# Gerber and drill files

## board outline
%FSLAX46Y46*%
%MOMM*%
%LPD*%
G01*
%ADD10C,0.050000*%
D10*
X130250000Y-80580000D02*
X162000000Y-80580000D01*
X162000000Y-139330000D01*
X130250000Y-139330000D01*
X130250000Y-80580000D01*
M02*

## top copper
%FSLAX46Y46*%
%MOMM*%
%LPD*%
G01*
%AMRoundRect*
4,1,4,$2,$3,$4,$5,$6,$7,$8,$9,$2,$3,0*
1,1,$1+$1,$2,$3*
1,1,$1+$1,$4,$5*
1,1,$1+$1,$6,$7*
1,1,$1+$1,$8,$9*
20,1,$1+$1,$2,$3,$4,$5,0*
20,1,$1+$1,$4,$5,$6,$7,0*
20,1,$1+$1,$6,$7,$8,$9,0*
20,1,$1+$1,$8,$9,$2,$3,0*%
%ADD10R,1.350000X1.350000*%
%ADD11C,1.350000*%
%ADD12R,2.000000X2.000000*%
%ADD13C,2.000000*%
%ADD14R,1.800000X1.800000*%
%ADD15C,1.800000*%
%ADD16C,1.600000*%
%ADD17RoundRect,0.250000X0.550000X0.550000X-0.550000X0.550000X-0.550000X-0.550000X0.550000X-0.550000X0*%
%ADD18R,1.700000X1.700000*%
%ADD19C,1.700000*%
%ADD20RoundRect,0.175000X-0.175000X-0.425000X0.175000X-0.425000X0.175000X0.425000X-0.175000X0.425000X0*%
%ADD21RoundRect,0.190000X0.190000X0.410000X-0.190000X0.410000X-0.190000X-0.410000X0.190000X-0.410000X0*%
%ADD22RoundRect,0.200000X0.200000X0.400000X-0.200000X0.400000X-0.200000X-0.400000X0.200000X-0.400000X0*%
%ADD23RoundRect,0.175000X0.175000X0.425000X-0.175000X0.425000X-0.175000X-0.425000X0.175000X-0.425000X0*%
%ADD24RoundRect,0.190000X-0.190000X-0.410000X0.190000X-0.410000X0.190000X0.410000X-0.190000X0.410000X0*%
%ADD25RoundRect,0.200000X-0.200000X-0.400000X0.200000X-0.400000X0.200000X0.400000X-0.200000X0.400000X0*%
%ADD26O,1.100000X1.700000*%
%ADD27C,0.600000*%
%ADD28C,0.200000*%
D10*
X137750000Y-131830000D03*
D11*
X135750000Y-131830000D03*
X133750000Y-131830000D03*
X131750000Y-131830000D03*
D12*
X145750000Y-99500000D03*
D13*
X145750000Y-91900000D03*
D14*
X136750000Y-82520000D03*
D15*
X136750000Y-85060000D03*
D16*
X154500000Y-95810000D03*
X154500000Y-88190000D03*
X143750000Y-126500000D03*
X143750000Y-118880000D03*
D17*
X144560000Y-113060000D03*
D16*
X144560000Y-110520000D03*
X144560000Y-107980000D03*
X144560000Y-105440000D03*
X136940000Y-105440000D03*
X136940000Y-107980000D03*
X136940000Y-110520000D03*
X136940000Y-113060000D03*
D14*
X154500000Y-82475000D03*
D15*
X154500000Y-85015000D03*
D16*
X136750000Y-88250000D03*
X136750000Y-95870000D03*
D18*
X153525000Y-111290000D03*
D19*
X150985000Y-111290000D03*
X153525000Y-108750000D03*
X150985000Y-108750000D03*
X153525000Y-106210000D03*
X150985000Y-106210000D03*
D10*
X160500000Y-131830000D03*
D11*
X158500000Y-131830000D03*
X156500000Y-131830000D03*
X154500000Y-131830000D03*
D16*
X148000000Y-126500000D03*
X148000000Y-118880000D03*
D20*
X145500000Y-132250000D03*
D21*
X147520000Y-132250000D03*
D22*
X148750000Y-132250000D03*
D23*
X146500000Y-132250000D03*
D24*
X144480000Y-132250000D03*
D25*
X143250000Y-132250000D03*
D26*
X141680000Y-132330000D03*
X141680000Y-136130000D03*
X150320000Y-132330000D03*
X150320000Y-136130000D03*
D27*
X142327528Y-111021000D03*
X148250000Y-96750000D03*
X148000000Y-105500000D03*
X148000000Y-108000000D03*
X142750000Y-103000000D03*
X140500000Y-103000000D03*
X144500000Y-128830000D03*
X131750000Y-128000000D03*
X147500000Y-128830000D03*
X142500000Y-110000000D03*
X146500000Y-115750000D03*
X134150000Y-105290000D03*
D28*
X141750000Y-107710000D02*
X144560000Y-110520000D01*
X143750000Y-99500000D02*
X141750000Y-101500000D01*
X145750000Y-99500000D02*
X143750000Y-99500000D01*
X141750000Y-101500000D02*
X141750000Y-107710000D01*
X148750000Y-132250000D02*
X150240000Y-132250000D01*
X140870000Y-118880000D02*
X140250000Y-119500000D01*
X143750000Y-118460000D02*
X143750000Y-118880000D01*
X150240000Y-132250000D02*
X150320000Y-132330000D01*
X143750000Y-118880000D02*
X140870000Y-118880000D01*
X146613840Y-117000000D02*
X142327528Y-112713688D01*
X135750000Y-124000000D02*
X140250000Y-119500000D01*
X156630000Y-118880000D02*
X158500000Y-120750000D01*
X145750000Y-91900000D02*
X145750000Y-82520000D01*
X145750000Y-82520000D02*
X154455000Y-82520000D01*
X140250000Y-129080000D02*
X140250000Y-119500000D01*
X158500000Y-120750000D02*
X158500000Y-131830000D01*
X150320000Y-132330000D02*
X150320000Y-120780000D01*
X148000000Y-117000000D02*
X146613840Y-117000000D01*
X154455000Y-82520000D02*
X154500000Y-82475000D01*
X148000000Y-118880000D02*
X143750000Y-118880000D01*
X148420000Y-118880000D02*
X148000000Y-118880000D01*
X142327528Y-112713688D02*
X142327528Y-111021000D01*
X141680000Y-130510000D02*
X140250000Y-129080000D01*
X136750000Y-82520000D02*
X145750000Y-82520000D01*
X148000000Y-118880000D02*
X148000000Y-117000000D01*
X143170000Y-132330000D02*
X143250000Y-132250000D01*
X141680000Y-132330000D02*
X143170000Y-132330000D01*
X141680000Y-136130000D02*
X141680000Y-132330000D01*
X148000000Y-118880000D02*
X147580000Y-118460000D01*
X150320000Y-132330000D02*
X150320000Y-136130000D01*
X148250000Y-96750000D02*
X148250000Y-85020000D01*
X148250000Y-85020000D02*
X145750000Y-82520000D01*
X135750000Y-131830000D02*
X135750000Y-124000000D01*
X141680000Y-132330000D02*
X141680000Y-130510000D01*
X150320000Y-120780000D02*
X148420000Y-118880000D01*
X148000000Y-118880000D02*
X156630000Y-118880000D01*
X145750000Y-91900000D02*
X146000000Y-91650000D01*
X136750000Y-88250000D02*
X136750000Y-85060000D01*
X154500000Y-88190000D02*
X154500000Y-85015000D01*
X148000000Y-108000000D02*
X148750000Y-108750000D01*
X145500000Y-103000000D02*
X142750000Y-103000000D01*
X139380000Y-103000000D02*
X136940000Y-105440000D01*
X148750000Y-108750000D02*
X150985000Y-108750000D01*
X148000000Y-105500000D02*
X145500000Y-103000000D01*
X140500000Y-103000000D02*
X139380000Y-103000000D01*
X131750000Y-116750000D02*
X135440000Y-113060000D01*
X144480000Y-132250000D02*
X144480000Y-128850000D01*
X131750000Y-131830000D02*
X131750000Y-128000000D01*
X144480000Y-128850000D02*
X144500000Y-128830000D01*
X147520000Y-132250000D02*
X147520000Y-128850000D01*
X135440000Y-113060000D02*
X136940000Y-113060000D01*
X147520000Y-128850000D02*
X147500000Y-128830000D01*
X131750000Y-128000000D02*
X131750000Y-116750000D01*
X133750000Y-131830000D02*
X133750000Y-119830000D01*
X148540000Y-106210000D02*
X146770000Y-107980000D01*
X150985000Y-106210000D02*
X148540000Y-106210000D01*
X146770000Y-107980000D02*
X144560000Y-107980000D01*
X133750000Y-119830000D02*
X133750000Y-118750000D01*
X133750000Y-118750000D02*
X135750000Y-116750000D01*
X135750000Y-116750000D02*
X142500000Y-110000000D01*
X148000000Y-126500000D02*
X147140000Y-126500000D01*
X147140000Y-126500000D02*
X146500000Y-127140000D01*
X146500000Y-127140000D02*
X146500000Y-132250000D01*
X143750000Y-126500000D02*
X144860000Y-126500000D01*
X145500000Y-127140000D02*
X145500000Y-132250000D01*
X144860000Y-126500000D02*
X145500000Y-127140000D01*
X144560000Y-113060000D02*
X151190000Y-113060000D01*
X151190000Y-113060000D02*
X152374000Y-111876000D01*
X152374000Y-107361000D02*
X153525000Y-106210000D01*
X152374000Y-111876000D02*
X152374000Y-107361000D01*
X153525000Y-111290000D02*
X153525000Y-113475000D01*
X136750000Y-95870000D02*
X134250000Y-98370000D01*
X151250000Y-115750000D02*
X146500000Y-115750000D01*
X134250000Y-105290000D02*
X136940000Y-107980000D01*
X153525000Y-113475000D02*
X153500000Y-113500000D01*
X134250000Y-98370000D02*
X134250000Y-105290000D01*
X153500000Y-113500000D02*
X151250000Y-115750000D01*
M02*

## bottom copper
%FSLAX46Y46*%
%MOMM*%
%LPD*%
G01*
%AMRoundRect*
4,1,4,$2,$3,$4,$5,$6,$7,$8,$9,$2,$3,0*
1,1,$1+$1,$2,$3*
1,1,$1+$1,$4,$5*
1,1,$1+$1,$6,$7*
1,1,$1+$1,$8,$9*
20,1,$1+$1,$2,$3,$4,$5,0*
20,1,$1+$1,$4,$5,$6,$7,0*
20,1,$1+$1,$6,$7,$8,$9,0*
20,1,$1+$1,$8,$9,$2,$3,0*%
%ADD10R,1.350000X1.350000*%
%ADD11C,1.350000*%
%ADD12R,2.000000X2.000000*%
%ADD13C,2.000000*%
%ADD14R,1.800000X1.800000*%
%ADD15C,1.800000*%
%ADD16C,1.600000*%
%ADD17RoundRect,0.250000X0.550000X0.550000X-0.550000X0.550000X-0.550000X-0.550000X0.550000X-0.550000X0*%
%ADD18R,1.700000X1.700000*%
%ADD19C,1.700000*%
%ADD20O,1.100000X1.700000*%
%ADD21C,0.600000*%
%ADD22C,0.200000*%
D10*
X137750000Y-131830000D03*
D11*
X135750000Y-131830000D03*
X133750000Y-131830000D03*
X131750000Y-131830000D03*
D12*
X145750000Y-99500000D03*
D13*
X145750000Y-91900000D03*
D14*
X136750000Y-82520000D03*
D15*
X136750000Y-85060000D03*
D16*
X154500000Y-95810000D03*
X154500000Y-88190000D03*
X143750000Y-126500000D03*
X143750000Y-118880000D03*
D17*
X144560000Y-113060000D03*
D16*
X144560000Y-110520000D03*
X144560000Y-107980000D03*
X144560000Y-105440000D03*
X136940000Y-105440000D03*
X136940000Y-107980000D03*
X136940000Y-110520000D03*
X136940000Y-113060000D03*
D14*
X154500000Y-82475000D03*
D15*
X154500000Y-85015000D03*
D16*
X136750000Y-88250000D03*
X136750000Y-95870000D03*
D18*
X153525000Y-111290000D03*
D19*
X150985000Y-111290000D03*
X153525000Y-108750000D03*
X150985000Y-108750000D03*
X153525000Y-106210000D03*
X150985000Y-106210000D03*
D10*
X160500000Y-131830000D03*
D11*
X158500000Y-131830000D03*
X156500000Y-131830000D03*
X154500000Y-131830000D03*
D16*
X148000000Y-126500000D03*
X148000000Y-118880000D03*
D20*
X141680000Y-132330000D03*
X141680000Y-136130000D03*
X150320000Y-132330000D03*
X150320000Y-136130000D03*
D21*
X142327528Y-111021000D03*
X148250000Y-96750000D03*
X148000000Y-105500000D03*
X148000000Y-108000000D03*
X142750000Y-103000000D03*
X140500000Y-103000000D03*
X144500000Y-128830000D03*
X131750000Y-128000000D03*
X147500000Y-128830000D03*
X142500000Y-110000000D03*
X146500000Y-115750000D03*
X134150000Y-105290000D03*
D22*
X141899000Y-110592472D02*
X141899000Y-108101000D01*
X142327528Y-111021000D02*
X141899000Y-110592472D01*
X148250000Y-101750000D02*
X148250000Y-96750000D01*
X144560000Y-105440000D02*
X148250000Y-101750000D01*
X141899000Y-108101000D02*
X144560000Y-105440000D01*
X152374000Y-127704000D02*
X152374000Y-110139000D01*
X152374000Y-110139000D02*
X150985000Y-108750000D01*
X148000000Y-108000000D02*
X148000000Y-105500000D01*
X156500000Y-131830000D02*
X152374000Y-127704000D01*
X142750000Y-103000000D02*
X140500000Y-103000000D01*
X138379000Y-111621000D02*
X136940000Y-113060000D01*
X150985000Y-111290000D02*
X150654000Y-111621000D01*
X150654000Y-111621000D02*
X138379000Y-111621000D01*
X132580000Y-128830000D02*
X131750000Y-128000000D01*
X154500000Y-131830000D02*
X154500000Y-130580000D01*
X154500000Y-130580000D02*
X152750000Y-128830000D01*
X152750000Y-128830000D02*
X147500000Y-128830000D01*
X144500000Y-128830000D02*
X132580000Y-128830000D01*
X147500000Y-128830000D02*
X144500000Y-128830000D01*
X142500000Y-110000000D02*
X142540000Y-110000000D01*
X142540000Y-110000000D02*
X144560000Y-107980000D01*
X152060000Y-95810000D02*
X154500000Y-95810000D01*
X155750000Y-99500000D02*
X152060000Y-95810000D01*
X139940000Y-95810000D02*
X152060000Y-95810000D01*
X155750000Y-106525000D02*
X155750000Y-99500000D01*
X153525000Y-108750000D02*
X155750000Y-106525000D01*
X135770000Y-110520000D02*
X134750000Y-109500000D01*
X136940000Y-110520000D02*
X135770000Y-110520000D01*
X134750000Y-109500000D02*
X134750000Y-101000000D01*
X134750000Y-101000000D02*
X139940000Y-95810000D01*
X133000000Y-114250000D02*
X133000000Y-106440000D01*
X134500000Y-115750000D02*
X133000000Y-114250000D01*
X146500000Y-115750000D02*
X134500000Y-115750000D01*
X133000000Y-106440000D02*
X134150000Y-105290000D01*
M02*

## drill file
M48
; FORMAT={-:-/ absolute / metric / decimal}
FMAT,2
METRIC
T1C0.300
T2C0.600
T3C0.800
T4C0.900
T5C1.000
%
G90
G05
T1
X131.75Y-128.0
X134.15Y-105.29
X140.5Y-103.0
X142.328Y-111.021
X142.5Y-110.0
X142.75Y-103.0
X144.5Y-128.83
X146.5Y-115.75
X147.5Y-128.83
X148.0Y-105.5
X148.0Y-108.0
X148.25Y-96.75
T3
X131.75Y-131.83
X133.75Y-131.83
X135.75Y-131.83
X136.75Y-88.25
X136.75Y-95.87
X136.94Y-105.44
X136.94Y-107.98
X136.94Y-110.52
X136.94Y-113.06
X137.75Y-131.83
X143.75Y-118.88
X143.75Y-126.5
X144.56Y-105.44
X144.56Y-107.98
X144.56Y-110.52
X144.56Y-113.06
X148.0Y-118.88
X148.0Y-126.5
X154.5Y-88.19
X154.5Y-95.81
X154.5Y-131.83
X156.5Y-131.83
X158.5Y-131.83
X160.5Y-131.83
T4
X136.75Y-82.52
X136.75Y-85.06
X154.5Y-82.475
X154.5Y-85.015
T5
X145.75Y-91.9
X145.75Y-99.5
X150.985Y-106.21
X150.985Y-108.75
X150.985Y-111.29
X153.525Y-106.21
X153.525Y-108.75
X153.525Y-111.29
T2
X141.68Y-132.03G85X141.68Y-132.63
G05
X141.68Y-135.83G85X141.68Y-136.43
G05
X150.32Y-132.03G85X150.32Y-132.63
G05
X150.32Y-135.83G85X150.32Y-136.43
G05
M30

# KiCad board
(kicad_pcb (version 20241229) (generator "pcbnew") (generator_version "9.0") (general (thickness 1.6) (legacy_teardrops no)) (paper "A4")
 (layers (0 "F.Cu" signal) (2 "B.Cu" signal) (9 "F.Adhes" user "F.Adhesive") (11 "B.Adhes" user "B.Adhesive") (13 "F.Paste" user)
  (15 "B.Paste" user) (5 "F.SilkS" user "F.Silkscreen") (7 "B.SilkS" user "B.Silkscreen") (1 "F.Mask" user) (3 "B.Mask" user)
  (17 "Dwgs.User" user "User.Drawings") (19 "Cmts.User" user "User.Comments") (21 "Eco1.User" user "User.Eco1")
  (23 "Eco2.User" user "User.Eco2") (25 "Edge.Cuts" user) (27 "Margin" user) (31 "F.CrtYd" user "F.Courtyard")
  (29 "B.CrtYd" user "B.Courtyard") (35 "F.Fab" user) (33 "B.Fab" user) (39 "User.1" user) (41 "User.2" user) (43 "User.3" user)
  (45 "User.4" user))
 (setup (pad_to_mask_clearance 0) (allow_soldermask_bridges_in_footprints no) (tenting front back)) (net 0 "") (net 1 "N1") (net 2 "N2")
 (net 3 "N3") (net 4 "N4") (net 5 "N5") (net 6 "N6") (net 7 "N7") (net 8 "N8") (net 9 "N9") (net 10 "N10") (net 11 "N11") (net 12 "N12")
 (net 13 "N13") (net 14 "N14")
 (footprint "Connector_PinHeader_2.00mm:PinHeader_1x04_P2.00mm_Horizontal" (layer "F.Cu") (at 137.75 131.83 -90)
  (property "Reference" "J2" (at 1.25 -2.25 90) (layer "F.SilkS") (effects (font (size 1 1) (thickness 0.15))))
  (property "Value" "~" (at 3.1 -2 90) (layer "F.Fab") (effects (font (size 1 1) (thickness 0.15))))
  (pad "1" thru_hole rect (at 0 0 270) (size 1.35 1.35) (drill 0.8) (layers "*.Cu" "*.Mask") (remove_unused_layers no) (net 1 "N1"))
  (pad "2" thru_hole circle (at 0 2 270) (size 1.35 1.35) (drill 0.8) (layers "*.Cu" "*.Mask") (remove_unused_layers no) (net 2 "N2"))
  (pad "3" thru_hole circle (at 0 4 270) (size 1.35 1.35) (drill 0.8) (layers "*.Cu" "*.Mask") (remove_unused_layers no) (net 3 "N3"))
  (pad "4" thru_hole circle (at 0 6 270) (size 1.35 1.35) (drill 0.8) (layers "*.Cu" "*.Mask") (remove_unused_layers no) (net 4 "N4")))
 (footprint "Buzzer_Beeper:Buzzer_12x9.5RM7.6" (layer "F.Cu") (at 145.75 99.5 90)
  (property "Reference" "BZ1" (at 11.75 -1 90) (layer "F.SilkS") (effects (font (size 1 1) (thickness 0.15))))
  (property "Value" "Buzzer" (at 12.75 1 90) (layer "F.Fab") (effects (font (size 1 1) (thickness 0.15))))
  (pad "1" thru_hole rect (at 0 0 90) (size 2 2) (drill 1) (layers "*.Cu" "*.Mask") (remove_unused_layers no) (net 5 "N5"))
  (pad "2" thru_hole circle (at 7.6 0 90) (size 2 2) (drill 1) (layers "*.Cu" "*.Mask") (remove_unused_layers no) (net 2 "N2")))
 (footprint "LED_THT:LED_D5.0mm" (layer "F.Cu") (at 136.75 82.52 -90)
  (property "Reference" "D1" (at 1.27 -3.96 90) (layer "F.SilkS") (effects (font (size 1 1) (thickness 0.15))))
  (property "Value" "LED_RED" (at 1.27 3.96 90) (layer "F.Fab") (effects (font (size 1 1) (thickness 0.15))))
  (pad "1" thru_hole rect (at 0 0 270) (size 1.8 1.8) (drill 0.9) (layers "*.Cu" "*.Mask") (remove_unused_layers no) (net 2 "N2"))
  (pad "2" thru_hole circle (at 2.54 0 270) (size 1.8 1.8) (drill 0.9) (layers "*.Cu" "*.Mask") (remove_unused_layers no) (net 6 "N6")))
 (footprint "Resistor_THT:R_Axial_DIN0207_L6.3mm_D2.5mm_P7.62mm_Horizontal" (layer "F.Cu") (at 154.5 95.81 90)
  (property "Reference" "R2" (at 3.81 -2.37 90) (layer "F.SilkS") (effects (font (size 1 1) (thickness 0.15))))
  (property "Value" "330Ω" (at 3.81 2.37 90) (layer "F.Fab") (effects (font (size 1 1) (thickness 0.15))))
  (pad "1" thru_hole circle (at 0 0 90) (size 1.6 1.6) (drill 0.8) (layers "*.Cu" "*.Mask") (remove_unused_layers no) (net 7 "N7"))
  (pad "2" thru_hole circle (at 7.62 0 90) (size 1.6 1.6) (drill 0.8) (layers "*.Cu" "*.Mask") (remove_unused_layers no) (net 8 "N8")))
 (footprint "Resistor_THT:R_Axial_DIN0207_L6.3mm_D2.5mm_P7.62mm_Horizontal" (layer "F.Cu") (at 143.75 126.5 90)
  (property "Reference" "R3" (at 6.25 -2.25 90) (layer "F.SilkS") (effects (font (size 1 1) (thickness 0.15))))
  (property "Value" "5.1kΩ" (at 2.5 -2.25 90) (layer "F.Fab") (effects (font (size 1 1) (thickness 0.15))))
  (pad "1" thru_hole circle (at 0 0 90) (size 1.6 1.6) (drill 0.8) (layers "*.Cu" "*.Mask") (remove_unused_layers no) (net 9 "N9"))
  (pad "2" thru_hole circle (at 7.62 0 90) (size 1.6 1.6) (drill 0.8) (layers "*.Cu" "*.Mask") (remove_unused_layers no) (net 2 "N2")))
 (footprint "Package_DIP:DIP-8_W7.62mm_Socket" (layer "F.Cu") (at 144.56 113.06 180)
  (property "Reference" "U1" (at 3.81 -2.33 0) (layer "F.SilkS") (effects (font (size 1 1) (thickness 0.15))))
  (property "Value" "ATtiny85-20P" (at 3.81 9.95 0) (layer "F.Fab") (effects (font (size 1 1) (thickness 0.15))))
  (pad "1" thru_hole roundrect (at 0 0 180) (size 1.6 1.6) (drill 0.8) (layers "*.Cu" "*.Mask") (remove_unused_layers no)
   (roundrect_rratio 0.15625) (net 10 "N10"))
  (pad "2" thru_hole circle (at 0 2.54 180) (size 1.6 1.6) (drill 0.8) (layers "*.Cu" "*.Mask") (remove_unused_layers no) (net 5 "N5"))
  (pad "3" thru_hole circle (at 0 5.08 180) (size 1.6 1.6) (drill 0.8) (layers "*.Cu" "*.Mask") (remove_unused_layers no) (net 3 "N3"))
  (pad "4" thru_hole circle (at 0 7.62 180) (size 1.6 1.6) (drill 0.8) (layers "*.Cu" "*.Mask") (remove_unused_layers no) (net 2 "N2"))
  (pad "5" thru_hole circle (at 7.62 7.62 180) (size 1.6 1.6) (drill 0.8) (layers "*.Cu" "*.Mask") (remove_unused_layers no) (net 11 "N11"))
  (pad "6" thru_hole circle (at 7.62 5.08 180) (size 1.6 1.6) (drill 0.8) (layers "*.Cu" "*.Mask") (remove_unused_layers no) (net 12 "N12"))
  (pad "7" thru_hole circle (at 7.62 2.54 180) (size 1.6 1.6) (drill 0.8) (layers "*.Cu" "*.Mask") (remove_unused_layers no) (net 7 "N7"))
  (pad "8" thru_hole circle (at 7.62 0 180) (size 1.6 1.6) (drill 0.8) (layers "*.Cu" "*.Mask") (remove_unused_layers no) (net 4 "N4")))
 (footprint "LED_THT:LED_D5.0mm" (layer "F.Cu") (at 154.5 82.475 -90)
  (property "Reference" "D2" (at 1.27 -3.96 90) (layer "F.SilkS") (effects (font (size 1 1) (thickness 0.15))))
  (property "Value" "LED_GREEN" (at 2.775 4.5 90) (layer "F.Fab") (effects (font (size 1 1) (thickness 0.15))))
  (pad "1" thru_hole rect (at 0 0 270) (size 1.8 1.8) (drill 0.9) (layers "*.Cu" "*.Mask") (remove_unused_layers no) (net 2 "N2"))
  (pad "2" thru_hole circle (at 2.54 0 270) (size 1.8 1.8) (drill 0.9) (layers "*.Cu" "*.Mask") (remove_unused_layers no) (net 8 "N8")))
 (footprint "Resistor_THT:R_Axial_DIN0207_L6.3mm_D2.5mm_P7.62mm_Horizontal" (layer "F.Cu") (at 136.75 88.25 -90)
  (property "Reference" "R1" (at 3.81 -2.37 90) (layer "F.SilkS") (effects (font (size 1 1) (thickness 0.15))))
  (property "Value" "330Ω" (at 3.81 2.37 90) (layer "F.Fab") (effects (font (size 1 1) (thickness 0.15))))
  (pad "1" thru_hole circle (at 0 0 270) (size 1.6 1.6) (drill 0.8) (layers "*.Cu" "*.Mask") (remove_unused_layers no) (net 6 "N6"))
  (pad "2" thru_hole circle (at 7.62 0 270) (size 1.6 1.6) (drill 0.8) (layers "*.Cu" "*.Mask") (remove_unused_layers no) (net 12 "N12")))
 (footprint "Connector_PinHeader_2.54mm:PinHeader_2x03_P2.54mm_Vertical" (layer "F.Cu") (at 153.525 111.29 180)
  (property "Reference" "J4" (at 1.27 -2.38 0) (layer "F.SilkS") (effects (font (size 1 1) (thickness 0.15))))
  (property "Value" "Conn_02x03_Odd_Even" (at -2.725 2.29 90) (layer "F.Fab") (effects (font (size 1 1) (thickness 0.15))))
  (pad "1" thru_hole rect (at 0 0 180) (size 1.7 1.7) (drill 1) (layers "*.Cu" "*.Mask") (remove_unused_layers no) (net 12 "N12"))
  (pad "2" thru_hole circle (at 2.54 0 180) (size 1.7 1.7) (drill 1) (layers "*.Cu" "*.Mask") (remove_unused_layers no) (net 4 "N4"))
  (pad "3" thru_hole circle (at 0 2.54 180) (size 1.7 1.7) (drill 1) (layers "*.Cu" "*.Mask") (remove_unused_layers no) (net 7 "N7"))
  (pad "4" thru_hole circle (at 2.54 2.54 180) (size 1.7 1.7) (drill 1) (layers "*.Cu" "*.Mask") (remove_unused_layers no) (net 11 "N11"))
  (pad "5" thru_hole circle (at 0 5.08 180) (size 1.7 1.7) (drill 1) (layers "*.Cu" "*.Mask") (remove_unused_layers no) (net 10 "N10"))
  (pad "6" thru_hole circle (at 2.54 5.08 180) (size 1.7 1.7) (drill 1) (layers "*.Cu" "*.Mask") (remove_unused_layers no) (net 3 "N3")))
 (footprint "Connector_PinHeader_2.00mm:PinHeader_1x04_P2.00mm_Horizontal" (layer "F.Cu") (at 160.5 131.83 -90)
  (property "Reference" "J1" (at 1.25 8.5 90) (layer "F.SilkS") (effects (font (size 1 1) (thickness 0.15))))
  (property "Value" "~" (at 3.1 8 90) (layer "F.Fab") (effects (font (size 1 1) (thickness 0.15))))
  (pad "1" thru_hole rect (at 0 0 270) (size 1.35 1.35) (drill 0.8) (layers "*.Cu" "*.Mask") (remove_unused_layers no) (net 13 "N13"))
  (pad "2" thru_hole circle (at 0 2 270) (size 1.35 1.35) (drill 0.8) (layers "*.Cu" "*.Mask") (remove_unused_layers no) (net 2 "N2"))
  (pad "3" thru_hole circle (at 0 4 270) (size 1.35 1.35) (drill 0.8) (layers "*.Cu" "*.Mask") (remove_unused_layers no) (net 11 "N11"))
  (pad "4" thru_hole circle (at 0 6 270) (size 1.35 1.35) (drill 0.8) (layers "*.Cu" "*.Mask") (remove_unused_layers no) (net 4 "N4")))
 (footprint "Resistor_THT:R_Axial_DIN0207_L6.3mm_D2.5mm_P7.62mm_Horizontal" (layer "F.Cu") (at 148 126.5 90)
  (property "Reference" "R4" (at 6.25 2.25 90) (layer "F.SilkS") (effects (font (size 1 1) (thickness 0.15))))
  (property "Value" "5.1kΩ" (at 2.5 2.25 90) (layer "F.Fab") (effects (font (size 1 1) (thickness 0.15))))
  (pad "1" thru_hole circle (at 0 0 90) (size 1.6 1.6) (drill 0.8) (layers "*.Cu" "*.Mask") (remove_unused_layers no) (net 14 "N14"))
  (pad "2" thru_hole circle (at 7.62 0 90) (size 1.6 1.6) (drill 0.8) (layers "*.Cu" "*.Mask") (remove_unused_layers no) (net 2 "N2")))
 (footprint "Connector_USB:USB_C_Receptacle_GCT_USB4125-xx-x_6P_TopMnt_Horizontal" (layer "F.Cu") (at 146 135.33)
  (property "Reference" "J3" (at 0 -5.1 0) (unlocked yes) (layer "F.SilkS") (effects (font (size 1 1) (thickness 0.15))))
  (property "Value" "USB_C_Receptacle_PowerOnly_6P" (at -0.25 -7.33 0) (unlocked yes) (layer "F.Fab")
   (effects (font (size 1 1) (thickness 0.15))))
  (pad "A5" smd roundrect (at -0.5 -3.08) (size 0.7 1.2) (layers "F.Cu" "F.Mask" "F.Paste") (roundrect_rratio 0.25) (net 9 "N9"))
  (pad "A9" smd roundrect (at 1.52 -3.08 180) (size 0.76 1.2) (layers "F.Cu" "F.Mask" "F.Paste") (roundrect_rratio 0.25) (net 4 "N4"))
  (pad "A12" smd roundrect (at 2.75 -3.08 180) (size 0.8 1.2) (layers "F.Cu" "F.Mask" "F.Paste") (roundrect_rratio 0.25) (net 2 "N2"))
  (pad "B5" smd roundrect (at 0.5 -3.08 180) (size 0.7 1.2) (layers "F.Cu" "F.Mask" "F.Paste") (roundrect_rratio 0.25) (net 14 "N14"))
  (pad "B9" smd roundrect (at -1.52 -3.08) (size 0.76 1.2) (layers "F.Cu" "F.Mask" "F.Paste") (roundrect_rratio 0.25) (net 4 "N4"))
  (pad "B12" smd roundrect (at -2.75 -3.08) (size 0.8 1.2) (layers "F.Cu" "F.Mask" "F.Paste") (roundrect_rratio 0.25) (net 2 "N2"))
  (pad "S1" thru_hole oval (at -4.32 -3) (size 1.1 1.7) (drill oval 0.6 1.2) (layers "*.Cu" "*.Mask" "F.Paste") (remove_unused_layers no)
   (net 2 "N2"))
  (pad "S1" thru_hole oval (at -4.32 0.8) (size 1.1 1.7) (drill oval 0.6 1.2) (layers "*.Cu" "*.Mask" "F.Paste") (remove_unused_layers no)
   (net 2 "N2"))
  (pad "S1" thru_hole oval (at 4.32 -3) (size 1.1 1.7) (drill oval 0.6 1.2) (layers "*.Cu" "*.Mask" "F.Paste") (remove_unused_layers no)
   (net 2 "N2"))
  (pad "S1" thru_hole oval (at 4.32 0.8) (size 1.1 1.7) (drill oval 0.6 1.2) (layers "*.Cu" "*.Mask" "F.Paste") (remove_unused_layers no)
   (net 2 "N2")))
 (gr_rect (start 130.25 80.58) (end 162 139.33) (stroke (width 0.05) (type default)) (fill no) (layer "Edge.Cuts"))
 (segment (start 141.75 107.71) (end 144.56 110.52) (width 0.2) (layer "F.Cu") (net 5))
 (segment (start 143.75 99.5) (end 141.75 101.5) (width 0.2) (layer "F.Cu") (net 5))
 (segment (start 145.75 99.5) (end 143.75 99.5) (width 0.2) (layer "F.Cu") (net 5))
 (segment (start 141.75 101.5) (end 141.75 107.71) (width 0.2) (layer "F.Cu") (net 5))
 (segment (start 148.75 132.25) (end 150.24 132.25) (width 0.2) (layer "F.Cu") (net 2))
 (segment (start 140.87 118.88) (end 140.25 119.5) (width 0.2) (layer "F.Cu") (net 2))
 (segment (start 143.75 118.46) (end 143.75 118.88) (width 0.2) (layer "F.Cu") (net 2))
 (segment (start 150.24 132.25) (end 150.32 132.33) (width 0.2) (layer "F.Cu") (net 2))
 (segment (start 143.75 118.88) (end 140.87 118.88) (width 0.2) (layer "F.Cu") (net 2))
 (segment (start 146.61384 117) (end 142.327528 112.713688) (width 0.2) (layer "F.Cu") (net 2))
 (segment (start 135.75 124) (end 140.25 119.5) (width 0.2) (layer "F.Cu") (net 2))
 (segment (start 156.63 118.88) (end 158.5 120.75) (width 0.2) (layer "F.Cu") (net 2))
 (segment (start 145.75 91.9) (end 145.75 82.52) (width 0.2) (layer "F.Cu") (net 2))
 (segment (start 145.75 82.52) (end 154.455 82.52) (width 0.2) (layer "F.Cu") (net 2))
 (segment (start 140.25 129.08) (end 140.25 119.5) (width 0.2) (layer "F.Cu") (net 2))
 (segment (start 158.5 120.75) (end 158.5 131.83) (width 0.2) (layer "F.Cu") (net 2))
 (segment (start 150.32 132.33) (end 150.32 120.78) (width 0.2) (layer "F.Cu") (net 2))
 (segment (start 148 117) (end 146.61384 117) (width 0.2) (layer "F.Cu") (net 2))
 (segment (start 154.455 82.52) (end 154.5 82.475) (width 0.2) (layer "F.Cu") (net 2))
 (segment (start 148 118.88) (end 143.75 118.88) (width 0.2) (layer "F.Cu") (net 2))
 (segment (start 148.42 118.88) (end 148 118.88) (width 0.2) (layer "F.Cu") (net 2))
 (segment (start 142.327528 112.713688) (end 142.327528 111.021) (width 0.2) (layer "F.Cu") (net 2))
 (segment (start 141.68 130.51) (end 140.25 129.08) (width 0.2) (layer "F.Cu") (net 2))
 (segment (start 136.75 82.52) (end 145.75 82.52) (width 0.2) (layer "F.Cu") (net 2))
 (segment (start 148 118.88) (end 148 117) (width 0.2) (layer "F.Cu") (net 2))
 (segment (start 143.17 132.33) (end 143.25 132.25) (width 0.2) (layer "F.Cu") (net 2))
 (segment (start 141.68 132.33) (end 143.17 132.33) (width 0.2) (layer "F.Cu") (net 2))
 (segment (start 141.68 136.13) (end 141.68 132.33) (width 0.2) (layer "F.Cu") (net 2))
 (segment (start 148 118.88) (end 147.58 118.46) (width 0.2) (layer "F.Cu") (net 2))
 (segment (start 150.32 132.33) (end 150.32 136.13) (width 0.2) (layer "F.Cu") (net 2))
 (segment (start 148.25 96.75) (end 148.25 85.02) (width 0.2) (layer "F.Cu") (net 2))
 (segment (start 148.25 85.02) (end 145.75 82.52) (width 0.2) (layer "F.Cu") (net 2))
 (segment (start 135.75 131.83) (end 135.75 124) (width 0.2) (layer "F.Cu") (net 2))
 (segment (start 141.68 132.33) (end 141.68 130.51) (width 0.2) (layer "F.Cu") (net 2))
 (segment (start 150.32 120.78) (end 148.42 118.88) (width 0.2) (layer "F.Cu") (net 2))
 (segment (start 148 118.88) (end 156.63 118.88) (width 0.2) (layer "F.Cu") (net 2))
 (segment (start 145.75 91.9) (end 146 91.65) (width 0.2) (layer "F.Cu") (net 2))
 (via (at 142.327528 111.021) (size 0.6) (drill 0.3) (layers "F.Cu" "B.Cu") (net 2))
 (via (at 148.25 96.75) (size 0.6) (drill 0.3) (layers "F.Cu" "B.Cu") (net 2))
 (segment (start 141.899 110.592472) (end 141.899 108.101) (width 0.2) (layer "B.Cu") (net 2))
 (segment (start 142.327528 111.021) (end 141.899 110.592472) (width 0.2) (layer "B.Cu") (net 2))
 (segment (start 148.25 101.75) (end 148.25 96.75) (width 0.2) (layer "B.Cu") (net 2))
 (segment (start 144.56 105.44) (end 148.25 101.75) (width 0.2) (layer "B.Cu") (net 2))
 (segment (start 141.899 108.101) (end 144.56 105.44) (width 0.2) (layer "B.Cu") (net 2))
 (segment (start 136.75 88.25) (end 136.75 85.06) (width 0.2) (layer "F.Cu") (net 6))
 (segment (start 154.5 88.19) (end 154.5 85.015) (width 0.2) (layer "F.Cu") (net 8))
 (segment (start 148 108) (end 148.75 108.75) (width 0.2) (layer "F.Cu") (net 11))
 (segment (start 145.5 103) (end 142.75 103) (width 0.2) (layer "F.Cu") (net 11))
 (segment (start 139.38 103) (end 136.94 105.44) (width 0.2) (layer "F.Cu") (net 11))
 (segment (start 148.75 108.75) (end 150.985 108.75) (width 0.2) (layer "F.Cu") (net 11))
 (segment (start 148 105.5) (end 145.5 103) (width 0.2) (layer "F.Cu") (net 11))
 (segment (start 140.5 103) (end 139.38 103) (width 0.2) (layer "F.Cu") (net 11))
 (via (at 148 105.5) (size 0.6) (drill 0.3) (layers "F.Cu" "B.Cu") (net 11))
 (via (at 148 108) (size 0.6) (drill 0.3) (layers "F.Cu" "B.Cu") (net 11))
 (via (at 142.75 103) (size 0.6) (drill 0.3) (layers "F.Cu" "B.Cu") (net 11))
 (via (at 140.5 103) (size 0.6) (drill 0.3) (layers "F.Cu" "B.Cu") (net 11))
 (segment (start 152.374 127.704) (end 152.374 110.139) (width 0.2) (layer "B.Cu") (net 11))
 (segment (start 152.374 110.139) (end 150.985 108.75) (width 0.2) (layer "B.Cu") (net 11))
 (segment (start 148 108) (end 148 105.5) (width 0.2) (layer "B.Cu") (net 11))
 (segment (start 156.5 131.83) (end 152.374 127.704) (width 0.2) (layer "B.Cu") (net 11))
 (segment (start 142.75 103) (end 140.5 103) (width 0.2) (layer "B.Cu") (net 11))
 (segment (start 131.75 116.75) (end 135.44 113.06) (width 0.2) (layer "F.Cu") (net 4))
 (segment (start 144.48 132.25) (end 144.48 128.85) (width 0.2) (layer "F.Cu") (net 4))
 (segment (start 131.75 131.83) (end 131.75 128) (width 0.2) (layer "F.Cu") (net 4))
 (segment (start 144.48 128.85) (end 144.5 128.83) (width 0.2) (layer "F.Cu") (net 4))
 (segment (start 147.52 132.25) (end 147.52 128.85) (width 0.2) (layer "F.Cu") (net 4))
 (segment (start 135.44 113.06) (end 136.94 113.06) (width 0.2) (layer "F.Cu") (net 4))
 (segment (start 147.52 128.85) (end 147.5 128.83) (width 0.2) (layer "F.Cu") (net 4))
 (segment (start 131.75 128) (end 131.75 116.75) (width 0.2) (layer "F.Cu") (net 4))
 (via (at 144.5 128.83) (size 0.6) (drill 0.3) (layers "F.Cu" "B.Cu") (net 4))
 (via (at 131.75 128) (size 0.6) (drill 0.3) (layers "F.Cu" "B.Cu") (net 4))
 (via (at 147.5 128.83) (size 0.6) (drill 0.3) (layers "F.Cu" "B.Cu") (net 4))
 (segment (start 138.379 111.621) (end 136.94 113.06) (width 0.2) (layer "B.Cu") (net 4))
 (segment (start 150.985 111.29) (end 150.654 111.621) (width 0.2) (layer "B.Cu") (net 4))
 (segment (start 150.654 111.621) (end 138.379 111.621) (width 0.2) (layer "B.Cu") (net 4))
 (segment (start 132.58 128.83) (end 131.75 128) (width 0.2) (layer "B.Cu") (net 4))
 (segment (start 154.5 131.83) (end 154.5 130.58) (width 0.2) (layer "B.Cu") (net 4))
 (segment (start 154.5 130.58) (end 152.75 128.83) (width 0.2) (layer "B.Cu") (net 4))
 (segment (start 152.75 128.83) (end 147.5 128.83) (width 0.2) (layer "B.Cu") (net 4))
 (segment (start 144.5 128.83) (end 132.58 128.83) (width 0.2) (layer "B.Cu") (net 4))
 (segment (start 147.5 128.83) (end 144.5 128.83) (width 0.2) (layer "B.Cu") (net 4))
 (segment (start 133.75 131.83) (end 133.75 119.83) (width 0.2) (layer "F.Cu") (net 3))
 (segment (start 148.54 106.21) (end 146.77 107.98) (width 0.2) (layer "F.Cu") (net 3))
 (segment (start 150.985 106.21) (end 148.54 106.21) (width 0.2) (layer "F.Cu") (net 3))
 (segment (start 146.77 107.98) (end 144.56 107.98) (width 0.2) (layer "F.Cu") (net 3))
 (segment (start 133.75 119.83) (end 133.75 118.75) (width 0.2) (layer "F.Cu") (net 3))
 (segment (start 133.75 118.75) (end 135.75 116.75) (width 0.2) (layer "F.Cu") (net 3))
 (segment (start 135.75 116.75) (end 142.5 110) (width 0.2) (layer "F.Cu") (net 3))
 (via (at 142.5 110) (size 0.6) (drill 0.3) (layers "F.Cu" "B.Cu") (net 3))
 (segment (start 142.5 110) (end 142.54 110) (width 0.2) (layer "B.Cu") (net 3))
 (segment (start 142.54 110) (end 144.56 107.98) (width 0.2) (layer "B.Cu") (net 3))
 (segment (start 148 126.5) (end 147.14 126.5) (width 0.2) (layer "F.Cu") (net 14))
 (segment (start 147.14 126.5) (end 146.5 127.14) (width 0.2) (layer "F.Cu") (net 14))
 (segment (start 146.5 127.14) (end 146.5 132.25) (width 0.2) (layer "F.Cu") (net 14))
 (segment (start 143.75 126.5) (end 144.86 126.5) (width 0.2) (layer "F.Cu") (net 9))
 (segment (start 145.5 127.14) (end 145.5 132.25) (width 0.2) (layer "F.Cu") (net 9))
 (segment (start 144.86 126.5) (end 145.5 127.14) (width 0.2) (layer "F.Cu") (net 9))
 (segment (start 152.06 95.81) (end 154.5 95.81) (width 0.2) (layer "B.Cu") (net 7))
 (segment (start 155.75 99.5) (end 152.06 95.81) (width 0.2) (layer "B.Cu") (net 7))
 (segment (start 139.94 95.81) (end 152.06 95.81) (width 0.2) (layer "B.Cu") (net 7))
 (segment (start 155.75 106.525) (end 155.75 99.5) (width 0.2) (layer "B.Cu") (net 7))
 (segment (start 153.525 108.75) (end 155.75 106.525) (width 0.2) (layer "B.Cu") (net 7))
 (segment (start 135.77 110.52) (end 134.75 109.5) (width 0.2) (layer "B.Cu") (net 7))
 (segment (start 136.94 110.52) (end 135.77 110.52) (width 0.2) (layer "B.Cu") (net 7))
 (segment (start 134.75 109.5) (end 134.75 101) (width 0.2) (layer "B.Cu") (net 7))
 (segment (start 134.75 101) (end 139.94 95.81) (width 0.2) (layer "B.Cu") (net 7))
 (segment (start 144.56 113.06) (end 151.19 113.06) (width 0.2) (layer "F.Cu") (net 10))
 (segment (start 151.19 113.06) (end 152.374 111.876) (width 0.2) (layer "F.Cu") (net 10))
 (segment (start 152.374 107.361) (end 153.525 106.21) (width 0.2) (layer "F.Cu") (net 10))
 (segment (start 152.374 111.876) (end 152.374 107.361) (width 0.2) (layer "F.Cu") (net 10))
 (segment (start 153.525 111.29) (end 153.525 113.475) (width 0.2) (layer "F.Cu") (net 12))
 (segment (start 136.75 95.87) (end 134.25 98.37) (width 0.2) (layer "F.Cu") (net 12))
 (segment (start 151.25 115.75) (end 146.5 115.75) (width 0.2) (layer "F.Cu") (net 12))
 (segment (start 134.25 105.29) (end 136.94 107.98) (width 0.2) (layer "F.Cu") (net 12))
 (segment (start 153.525 113.475) (end 153.5 113.5) (width 0.2) (layer "F.Cu") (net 12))
 (segment (start 134.25 98.37) (end 134.25 105.29) (width 0.2) (layer "F.Cu") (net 12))
 (segment (start 153.5 113.5) (end 151.25 115.75) (width 0.2) (layer "F.Cu") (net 12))
 (via (at 146.5 115.75) (size 0.6) (drill 0.3) (layers "F.Cu" "B.Cu") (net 12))
 (via (at 134.15 105.29) (size 0.6) (drill 0.3) (layers "F.Cu" "B.Cu") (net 12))
 (segment (start 133 114.25) (end 133 106.44) (width 0.2) (layer "B.Cu") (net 12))
 (segment (start 134.5 115.75) (end 133 114.25) (width 0.2) (layer "B.Cu") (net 12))
 (segment (start 146.5 115.75) (end 134.5 115.75) (width 0.2) (layer "B.Cu") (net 12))
 (segment (start 133 106.44) (end 134.15 105.29) (width 0.2) (layer "B.Cu") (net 12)))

